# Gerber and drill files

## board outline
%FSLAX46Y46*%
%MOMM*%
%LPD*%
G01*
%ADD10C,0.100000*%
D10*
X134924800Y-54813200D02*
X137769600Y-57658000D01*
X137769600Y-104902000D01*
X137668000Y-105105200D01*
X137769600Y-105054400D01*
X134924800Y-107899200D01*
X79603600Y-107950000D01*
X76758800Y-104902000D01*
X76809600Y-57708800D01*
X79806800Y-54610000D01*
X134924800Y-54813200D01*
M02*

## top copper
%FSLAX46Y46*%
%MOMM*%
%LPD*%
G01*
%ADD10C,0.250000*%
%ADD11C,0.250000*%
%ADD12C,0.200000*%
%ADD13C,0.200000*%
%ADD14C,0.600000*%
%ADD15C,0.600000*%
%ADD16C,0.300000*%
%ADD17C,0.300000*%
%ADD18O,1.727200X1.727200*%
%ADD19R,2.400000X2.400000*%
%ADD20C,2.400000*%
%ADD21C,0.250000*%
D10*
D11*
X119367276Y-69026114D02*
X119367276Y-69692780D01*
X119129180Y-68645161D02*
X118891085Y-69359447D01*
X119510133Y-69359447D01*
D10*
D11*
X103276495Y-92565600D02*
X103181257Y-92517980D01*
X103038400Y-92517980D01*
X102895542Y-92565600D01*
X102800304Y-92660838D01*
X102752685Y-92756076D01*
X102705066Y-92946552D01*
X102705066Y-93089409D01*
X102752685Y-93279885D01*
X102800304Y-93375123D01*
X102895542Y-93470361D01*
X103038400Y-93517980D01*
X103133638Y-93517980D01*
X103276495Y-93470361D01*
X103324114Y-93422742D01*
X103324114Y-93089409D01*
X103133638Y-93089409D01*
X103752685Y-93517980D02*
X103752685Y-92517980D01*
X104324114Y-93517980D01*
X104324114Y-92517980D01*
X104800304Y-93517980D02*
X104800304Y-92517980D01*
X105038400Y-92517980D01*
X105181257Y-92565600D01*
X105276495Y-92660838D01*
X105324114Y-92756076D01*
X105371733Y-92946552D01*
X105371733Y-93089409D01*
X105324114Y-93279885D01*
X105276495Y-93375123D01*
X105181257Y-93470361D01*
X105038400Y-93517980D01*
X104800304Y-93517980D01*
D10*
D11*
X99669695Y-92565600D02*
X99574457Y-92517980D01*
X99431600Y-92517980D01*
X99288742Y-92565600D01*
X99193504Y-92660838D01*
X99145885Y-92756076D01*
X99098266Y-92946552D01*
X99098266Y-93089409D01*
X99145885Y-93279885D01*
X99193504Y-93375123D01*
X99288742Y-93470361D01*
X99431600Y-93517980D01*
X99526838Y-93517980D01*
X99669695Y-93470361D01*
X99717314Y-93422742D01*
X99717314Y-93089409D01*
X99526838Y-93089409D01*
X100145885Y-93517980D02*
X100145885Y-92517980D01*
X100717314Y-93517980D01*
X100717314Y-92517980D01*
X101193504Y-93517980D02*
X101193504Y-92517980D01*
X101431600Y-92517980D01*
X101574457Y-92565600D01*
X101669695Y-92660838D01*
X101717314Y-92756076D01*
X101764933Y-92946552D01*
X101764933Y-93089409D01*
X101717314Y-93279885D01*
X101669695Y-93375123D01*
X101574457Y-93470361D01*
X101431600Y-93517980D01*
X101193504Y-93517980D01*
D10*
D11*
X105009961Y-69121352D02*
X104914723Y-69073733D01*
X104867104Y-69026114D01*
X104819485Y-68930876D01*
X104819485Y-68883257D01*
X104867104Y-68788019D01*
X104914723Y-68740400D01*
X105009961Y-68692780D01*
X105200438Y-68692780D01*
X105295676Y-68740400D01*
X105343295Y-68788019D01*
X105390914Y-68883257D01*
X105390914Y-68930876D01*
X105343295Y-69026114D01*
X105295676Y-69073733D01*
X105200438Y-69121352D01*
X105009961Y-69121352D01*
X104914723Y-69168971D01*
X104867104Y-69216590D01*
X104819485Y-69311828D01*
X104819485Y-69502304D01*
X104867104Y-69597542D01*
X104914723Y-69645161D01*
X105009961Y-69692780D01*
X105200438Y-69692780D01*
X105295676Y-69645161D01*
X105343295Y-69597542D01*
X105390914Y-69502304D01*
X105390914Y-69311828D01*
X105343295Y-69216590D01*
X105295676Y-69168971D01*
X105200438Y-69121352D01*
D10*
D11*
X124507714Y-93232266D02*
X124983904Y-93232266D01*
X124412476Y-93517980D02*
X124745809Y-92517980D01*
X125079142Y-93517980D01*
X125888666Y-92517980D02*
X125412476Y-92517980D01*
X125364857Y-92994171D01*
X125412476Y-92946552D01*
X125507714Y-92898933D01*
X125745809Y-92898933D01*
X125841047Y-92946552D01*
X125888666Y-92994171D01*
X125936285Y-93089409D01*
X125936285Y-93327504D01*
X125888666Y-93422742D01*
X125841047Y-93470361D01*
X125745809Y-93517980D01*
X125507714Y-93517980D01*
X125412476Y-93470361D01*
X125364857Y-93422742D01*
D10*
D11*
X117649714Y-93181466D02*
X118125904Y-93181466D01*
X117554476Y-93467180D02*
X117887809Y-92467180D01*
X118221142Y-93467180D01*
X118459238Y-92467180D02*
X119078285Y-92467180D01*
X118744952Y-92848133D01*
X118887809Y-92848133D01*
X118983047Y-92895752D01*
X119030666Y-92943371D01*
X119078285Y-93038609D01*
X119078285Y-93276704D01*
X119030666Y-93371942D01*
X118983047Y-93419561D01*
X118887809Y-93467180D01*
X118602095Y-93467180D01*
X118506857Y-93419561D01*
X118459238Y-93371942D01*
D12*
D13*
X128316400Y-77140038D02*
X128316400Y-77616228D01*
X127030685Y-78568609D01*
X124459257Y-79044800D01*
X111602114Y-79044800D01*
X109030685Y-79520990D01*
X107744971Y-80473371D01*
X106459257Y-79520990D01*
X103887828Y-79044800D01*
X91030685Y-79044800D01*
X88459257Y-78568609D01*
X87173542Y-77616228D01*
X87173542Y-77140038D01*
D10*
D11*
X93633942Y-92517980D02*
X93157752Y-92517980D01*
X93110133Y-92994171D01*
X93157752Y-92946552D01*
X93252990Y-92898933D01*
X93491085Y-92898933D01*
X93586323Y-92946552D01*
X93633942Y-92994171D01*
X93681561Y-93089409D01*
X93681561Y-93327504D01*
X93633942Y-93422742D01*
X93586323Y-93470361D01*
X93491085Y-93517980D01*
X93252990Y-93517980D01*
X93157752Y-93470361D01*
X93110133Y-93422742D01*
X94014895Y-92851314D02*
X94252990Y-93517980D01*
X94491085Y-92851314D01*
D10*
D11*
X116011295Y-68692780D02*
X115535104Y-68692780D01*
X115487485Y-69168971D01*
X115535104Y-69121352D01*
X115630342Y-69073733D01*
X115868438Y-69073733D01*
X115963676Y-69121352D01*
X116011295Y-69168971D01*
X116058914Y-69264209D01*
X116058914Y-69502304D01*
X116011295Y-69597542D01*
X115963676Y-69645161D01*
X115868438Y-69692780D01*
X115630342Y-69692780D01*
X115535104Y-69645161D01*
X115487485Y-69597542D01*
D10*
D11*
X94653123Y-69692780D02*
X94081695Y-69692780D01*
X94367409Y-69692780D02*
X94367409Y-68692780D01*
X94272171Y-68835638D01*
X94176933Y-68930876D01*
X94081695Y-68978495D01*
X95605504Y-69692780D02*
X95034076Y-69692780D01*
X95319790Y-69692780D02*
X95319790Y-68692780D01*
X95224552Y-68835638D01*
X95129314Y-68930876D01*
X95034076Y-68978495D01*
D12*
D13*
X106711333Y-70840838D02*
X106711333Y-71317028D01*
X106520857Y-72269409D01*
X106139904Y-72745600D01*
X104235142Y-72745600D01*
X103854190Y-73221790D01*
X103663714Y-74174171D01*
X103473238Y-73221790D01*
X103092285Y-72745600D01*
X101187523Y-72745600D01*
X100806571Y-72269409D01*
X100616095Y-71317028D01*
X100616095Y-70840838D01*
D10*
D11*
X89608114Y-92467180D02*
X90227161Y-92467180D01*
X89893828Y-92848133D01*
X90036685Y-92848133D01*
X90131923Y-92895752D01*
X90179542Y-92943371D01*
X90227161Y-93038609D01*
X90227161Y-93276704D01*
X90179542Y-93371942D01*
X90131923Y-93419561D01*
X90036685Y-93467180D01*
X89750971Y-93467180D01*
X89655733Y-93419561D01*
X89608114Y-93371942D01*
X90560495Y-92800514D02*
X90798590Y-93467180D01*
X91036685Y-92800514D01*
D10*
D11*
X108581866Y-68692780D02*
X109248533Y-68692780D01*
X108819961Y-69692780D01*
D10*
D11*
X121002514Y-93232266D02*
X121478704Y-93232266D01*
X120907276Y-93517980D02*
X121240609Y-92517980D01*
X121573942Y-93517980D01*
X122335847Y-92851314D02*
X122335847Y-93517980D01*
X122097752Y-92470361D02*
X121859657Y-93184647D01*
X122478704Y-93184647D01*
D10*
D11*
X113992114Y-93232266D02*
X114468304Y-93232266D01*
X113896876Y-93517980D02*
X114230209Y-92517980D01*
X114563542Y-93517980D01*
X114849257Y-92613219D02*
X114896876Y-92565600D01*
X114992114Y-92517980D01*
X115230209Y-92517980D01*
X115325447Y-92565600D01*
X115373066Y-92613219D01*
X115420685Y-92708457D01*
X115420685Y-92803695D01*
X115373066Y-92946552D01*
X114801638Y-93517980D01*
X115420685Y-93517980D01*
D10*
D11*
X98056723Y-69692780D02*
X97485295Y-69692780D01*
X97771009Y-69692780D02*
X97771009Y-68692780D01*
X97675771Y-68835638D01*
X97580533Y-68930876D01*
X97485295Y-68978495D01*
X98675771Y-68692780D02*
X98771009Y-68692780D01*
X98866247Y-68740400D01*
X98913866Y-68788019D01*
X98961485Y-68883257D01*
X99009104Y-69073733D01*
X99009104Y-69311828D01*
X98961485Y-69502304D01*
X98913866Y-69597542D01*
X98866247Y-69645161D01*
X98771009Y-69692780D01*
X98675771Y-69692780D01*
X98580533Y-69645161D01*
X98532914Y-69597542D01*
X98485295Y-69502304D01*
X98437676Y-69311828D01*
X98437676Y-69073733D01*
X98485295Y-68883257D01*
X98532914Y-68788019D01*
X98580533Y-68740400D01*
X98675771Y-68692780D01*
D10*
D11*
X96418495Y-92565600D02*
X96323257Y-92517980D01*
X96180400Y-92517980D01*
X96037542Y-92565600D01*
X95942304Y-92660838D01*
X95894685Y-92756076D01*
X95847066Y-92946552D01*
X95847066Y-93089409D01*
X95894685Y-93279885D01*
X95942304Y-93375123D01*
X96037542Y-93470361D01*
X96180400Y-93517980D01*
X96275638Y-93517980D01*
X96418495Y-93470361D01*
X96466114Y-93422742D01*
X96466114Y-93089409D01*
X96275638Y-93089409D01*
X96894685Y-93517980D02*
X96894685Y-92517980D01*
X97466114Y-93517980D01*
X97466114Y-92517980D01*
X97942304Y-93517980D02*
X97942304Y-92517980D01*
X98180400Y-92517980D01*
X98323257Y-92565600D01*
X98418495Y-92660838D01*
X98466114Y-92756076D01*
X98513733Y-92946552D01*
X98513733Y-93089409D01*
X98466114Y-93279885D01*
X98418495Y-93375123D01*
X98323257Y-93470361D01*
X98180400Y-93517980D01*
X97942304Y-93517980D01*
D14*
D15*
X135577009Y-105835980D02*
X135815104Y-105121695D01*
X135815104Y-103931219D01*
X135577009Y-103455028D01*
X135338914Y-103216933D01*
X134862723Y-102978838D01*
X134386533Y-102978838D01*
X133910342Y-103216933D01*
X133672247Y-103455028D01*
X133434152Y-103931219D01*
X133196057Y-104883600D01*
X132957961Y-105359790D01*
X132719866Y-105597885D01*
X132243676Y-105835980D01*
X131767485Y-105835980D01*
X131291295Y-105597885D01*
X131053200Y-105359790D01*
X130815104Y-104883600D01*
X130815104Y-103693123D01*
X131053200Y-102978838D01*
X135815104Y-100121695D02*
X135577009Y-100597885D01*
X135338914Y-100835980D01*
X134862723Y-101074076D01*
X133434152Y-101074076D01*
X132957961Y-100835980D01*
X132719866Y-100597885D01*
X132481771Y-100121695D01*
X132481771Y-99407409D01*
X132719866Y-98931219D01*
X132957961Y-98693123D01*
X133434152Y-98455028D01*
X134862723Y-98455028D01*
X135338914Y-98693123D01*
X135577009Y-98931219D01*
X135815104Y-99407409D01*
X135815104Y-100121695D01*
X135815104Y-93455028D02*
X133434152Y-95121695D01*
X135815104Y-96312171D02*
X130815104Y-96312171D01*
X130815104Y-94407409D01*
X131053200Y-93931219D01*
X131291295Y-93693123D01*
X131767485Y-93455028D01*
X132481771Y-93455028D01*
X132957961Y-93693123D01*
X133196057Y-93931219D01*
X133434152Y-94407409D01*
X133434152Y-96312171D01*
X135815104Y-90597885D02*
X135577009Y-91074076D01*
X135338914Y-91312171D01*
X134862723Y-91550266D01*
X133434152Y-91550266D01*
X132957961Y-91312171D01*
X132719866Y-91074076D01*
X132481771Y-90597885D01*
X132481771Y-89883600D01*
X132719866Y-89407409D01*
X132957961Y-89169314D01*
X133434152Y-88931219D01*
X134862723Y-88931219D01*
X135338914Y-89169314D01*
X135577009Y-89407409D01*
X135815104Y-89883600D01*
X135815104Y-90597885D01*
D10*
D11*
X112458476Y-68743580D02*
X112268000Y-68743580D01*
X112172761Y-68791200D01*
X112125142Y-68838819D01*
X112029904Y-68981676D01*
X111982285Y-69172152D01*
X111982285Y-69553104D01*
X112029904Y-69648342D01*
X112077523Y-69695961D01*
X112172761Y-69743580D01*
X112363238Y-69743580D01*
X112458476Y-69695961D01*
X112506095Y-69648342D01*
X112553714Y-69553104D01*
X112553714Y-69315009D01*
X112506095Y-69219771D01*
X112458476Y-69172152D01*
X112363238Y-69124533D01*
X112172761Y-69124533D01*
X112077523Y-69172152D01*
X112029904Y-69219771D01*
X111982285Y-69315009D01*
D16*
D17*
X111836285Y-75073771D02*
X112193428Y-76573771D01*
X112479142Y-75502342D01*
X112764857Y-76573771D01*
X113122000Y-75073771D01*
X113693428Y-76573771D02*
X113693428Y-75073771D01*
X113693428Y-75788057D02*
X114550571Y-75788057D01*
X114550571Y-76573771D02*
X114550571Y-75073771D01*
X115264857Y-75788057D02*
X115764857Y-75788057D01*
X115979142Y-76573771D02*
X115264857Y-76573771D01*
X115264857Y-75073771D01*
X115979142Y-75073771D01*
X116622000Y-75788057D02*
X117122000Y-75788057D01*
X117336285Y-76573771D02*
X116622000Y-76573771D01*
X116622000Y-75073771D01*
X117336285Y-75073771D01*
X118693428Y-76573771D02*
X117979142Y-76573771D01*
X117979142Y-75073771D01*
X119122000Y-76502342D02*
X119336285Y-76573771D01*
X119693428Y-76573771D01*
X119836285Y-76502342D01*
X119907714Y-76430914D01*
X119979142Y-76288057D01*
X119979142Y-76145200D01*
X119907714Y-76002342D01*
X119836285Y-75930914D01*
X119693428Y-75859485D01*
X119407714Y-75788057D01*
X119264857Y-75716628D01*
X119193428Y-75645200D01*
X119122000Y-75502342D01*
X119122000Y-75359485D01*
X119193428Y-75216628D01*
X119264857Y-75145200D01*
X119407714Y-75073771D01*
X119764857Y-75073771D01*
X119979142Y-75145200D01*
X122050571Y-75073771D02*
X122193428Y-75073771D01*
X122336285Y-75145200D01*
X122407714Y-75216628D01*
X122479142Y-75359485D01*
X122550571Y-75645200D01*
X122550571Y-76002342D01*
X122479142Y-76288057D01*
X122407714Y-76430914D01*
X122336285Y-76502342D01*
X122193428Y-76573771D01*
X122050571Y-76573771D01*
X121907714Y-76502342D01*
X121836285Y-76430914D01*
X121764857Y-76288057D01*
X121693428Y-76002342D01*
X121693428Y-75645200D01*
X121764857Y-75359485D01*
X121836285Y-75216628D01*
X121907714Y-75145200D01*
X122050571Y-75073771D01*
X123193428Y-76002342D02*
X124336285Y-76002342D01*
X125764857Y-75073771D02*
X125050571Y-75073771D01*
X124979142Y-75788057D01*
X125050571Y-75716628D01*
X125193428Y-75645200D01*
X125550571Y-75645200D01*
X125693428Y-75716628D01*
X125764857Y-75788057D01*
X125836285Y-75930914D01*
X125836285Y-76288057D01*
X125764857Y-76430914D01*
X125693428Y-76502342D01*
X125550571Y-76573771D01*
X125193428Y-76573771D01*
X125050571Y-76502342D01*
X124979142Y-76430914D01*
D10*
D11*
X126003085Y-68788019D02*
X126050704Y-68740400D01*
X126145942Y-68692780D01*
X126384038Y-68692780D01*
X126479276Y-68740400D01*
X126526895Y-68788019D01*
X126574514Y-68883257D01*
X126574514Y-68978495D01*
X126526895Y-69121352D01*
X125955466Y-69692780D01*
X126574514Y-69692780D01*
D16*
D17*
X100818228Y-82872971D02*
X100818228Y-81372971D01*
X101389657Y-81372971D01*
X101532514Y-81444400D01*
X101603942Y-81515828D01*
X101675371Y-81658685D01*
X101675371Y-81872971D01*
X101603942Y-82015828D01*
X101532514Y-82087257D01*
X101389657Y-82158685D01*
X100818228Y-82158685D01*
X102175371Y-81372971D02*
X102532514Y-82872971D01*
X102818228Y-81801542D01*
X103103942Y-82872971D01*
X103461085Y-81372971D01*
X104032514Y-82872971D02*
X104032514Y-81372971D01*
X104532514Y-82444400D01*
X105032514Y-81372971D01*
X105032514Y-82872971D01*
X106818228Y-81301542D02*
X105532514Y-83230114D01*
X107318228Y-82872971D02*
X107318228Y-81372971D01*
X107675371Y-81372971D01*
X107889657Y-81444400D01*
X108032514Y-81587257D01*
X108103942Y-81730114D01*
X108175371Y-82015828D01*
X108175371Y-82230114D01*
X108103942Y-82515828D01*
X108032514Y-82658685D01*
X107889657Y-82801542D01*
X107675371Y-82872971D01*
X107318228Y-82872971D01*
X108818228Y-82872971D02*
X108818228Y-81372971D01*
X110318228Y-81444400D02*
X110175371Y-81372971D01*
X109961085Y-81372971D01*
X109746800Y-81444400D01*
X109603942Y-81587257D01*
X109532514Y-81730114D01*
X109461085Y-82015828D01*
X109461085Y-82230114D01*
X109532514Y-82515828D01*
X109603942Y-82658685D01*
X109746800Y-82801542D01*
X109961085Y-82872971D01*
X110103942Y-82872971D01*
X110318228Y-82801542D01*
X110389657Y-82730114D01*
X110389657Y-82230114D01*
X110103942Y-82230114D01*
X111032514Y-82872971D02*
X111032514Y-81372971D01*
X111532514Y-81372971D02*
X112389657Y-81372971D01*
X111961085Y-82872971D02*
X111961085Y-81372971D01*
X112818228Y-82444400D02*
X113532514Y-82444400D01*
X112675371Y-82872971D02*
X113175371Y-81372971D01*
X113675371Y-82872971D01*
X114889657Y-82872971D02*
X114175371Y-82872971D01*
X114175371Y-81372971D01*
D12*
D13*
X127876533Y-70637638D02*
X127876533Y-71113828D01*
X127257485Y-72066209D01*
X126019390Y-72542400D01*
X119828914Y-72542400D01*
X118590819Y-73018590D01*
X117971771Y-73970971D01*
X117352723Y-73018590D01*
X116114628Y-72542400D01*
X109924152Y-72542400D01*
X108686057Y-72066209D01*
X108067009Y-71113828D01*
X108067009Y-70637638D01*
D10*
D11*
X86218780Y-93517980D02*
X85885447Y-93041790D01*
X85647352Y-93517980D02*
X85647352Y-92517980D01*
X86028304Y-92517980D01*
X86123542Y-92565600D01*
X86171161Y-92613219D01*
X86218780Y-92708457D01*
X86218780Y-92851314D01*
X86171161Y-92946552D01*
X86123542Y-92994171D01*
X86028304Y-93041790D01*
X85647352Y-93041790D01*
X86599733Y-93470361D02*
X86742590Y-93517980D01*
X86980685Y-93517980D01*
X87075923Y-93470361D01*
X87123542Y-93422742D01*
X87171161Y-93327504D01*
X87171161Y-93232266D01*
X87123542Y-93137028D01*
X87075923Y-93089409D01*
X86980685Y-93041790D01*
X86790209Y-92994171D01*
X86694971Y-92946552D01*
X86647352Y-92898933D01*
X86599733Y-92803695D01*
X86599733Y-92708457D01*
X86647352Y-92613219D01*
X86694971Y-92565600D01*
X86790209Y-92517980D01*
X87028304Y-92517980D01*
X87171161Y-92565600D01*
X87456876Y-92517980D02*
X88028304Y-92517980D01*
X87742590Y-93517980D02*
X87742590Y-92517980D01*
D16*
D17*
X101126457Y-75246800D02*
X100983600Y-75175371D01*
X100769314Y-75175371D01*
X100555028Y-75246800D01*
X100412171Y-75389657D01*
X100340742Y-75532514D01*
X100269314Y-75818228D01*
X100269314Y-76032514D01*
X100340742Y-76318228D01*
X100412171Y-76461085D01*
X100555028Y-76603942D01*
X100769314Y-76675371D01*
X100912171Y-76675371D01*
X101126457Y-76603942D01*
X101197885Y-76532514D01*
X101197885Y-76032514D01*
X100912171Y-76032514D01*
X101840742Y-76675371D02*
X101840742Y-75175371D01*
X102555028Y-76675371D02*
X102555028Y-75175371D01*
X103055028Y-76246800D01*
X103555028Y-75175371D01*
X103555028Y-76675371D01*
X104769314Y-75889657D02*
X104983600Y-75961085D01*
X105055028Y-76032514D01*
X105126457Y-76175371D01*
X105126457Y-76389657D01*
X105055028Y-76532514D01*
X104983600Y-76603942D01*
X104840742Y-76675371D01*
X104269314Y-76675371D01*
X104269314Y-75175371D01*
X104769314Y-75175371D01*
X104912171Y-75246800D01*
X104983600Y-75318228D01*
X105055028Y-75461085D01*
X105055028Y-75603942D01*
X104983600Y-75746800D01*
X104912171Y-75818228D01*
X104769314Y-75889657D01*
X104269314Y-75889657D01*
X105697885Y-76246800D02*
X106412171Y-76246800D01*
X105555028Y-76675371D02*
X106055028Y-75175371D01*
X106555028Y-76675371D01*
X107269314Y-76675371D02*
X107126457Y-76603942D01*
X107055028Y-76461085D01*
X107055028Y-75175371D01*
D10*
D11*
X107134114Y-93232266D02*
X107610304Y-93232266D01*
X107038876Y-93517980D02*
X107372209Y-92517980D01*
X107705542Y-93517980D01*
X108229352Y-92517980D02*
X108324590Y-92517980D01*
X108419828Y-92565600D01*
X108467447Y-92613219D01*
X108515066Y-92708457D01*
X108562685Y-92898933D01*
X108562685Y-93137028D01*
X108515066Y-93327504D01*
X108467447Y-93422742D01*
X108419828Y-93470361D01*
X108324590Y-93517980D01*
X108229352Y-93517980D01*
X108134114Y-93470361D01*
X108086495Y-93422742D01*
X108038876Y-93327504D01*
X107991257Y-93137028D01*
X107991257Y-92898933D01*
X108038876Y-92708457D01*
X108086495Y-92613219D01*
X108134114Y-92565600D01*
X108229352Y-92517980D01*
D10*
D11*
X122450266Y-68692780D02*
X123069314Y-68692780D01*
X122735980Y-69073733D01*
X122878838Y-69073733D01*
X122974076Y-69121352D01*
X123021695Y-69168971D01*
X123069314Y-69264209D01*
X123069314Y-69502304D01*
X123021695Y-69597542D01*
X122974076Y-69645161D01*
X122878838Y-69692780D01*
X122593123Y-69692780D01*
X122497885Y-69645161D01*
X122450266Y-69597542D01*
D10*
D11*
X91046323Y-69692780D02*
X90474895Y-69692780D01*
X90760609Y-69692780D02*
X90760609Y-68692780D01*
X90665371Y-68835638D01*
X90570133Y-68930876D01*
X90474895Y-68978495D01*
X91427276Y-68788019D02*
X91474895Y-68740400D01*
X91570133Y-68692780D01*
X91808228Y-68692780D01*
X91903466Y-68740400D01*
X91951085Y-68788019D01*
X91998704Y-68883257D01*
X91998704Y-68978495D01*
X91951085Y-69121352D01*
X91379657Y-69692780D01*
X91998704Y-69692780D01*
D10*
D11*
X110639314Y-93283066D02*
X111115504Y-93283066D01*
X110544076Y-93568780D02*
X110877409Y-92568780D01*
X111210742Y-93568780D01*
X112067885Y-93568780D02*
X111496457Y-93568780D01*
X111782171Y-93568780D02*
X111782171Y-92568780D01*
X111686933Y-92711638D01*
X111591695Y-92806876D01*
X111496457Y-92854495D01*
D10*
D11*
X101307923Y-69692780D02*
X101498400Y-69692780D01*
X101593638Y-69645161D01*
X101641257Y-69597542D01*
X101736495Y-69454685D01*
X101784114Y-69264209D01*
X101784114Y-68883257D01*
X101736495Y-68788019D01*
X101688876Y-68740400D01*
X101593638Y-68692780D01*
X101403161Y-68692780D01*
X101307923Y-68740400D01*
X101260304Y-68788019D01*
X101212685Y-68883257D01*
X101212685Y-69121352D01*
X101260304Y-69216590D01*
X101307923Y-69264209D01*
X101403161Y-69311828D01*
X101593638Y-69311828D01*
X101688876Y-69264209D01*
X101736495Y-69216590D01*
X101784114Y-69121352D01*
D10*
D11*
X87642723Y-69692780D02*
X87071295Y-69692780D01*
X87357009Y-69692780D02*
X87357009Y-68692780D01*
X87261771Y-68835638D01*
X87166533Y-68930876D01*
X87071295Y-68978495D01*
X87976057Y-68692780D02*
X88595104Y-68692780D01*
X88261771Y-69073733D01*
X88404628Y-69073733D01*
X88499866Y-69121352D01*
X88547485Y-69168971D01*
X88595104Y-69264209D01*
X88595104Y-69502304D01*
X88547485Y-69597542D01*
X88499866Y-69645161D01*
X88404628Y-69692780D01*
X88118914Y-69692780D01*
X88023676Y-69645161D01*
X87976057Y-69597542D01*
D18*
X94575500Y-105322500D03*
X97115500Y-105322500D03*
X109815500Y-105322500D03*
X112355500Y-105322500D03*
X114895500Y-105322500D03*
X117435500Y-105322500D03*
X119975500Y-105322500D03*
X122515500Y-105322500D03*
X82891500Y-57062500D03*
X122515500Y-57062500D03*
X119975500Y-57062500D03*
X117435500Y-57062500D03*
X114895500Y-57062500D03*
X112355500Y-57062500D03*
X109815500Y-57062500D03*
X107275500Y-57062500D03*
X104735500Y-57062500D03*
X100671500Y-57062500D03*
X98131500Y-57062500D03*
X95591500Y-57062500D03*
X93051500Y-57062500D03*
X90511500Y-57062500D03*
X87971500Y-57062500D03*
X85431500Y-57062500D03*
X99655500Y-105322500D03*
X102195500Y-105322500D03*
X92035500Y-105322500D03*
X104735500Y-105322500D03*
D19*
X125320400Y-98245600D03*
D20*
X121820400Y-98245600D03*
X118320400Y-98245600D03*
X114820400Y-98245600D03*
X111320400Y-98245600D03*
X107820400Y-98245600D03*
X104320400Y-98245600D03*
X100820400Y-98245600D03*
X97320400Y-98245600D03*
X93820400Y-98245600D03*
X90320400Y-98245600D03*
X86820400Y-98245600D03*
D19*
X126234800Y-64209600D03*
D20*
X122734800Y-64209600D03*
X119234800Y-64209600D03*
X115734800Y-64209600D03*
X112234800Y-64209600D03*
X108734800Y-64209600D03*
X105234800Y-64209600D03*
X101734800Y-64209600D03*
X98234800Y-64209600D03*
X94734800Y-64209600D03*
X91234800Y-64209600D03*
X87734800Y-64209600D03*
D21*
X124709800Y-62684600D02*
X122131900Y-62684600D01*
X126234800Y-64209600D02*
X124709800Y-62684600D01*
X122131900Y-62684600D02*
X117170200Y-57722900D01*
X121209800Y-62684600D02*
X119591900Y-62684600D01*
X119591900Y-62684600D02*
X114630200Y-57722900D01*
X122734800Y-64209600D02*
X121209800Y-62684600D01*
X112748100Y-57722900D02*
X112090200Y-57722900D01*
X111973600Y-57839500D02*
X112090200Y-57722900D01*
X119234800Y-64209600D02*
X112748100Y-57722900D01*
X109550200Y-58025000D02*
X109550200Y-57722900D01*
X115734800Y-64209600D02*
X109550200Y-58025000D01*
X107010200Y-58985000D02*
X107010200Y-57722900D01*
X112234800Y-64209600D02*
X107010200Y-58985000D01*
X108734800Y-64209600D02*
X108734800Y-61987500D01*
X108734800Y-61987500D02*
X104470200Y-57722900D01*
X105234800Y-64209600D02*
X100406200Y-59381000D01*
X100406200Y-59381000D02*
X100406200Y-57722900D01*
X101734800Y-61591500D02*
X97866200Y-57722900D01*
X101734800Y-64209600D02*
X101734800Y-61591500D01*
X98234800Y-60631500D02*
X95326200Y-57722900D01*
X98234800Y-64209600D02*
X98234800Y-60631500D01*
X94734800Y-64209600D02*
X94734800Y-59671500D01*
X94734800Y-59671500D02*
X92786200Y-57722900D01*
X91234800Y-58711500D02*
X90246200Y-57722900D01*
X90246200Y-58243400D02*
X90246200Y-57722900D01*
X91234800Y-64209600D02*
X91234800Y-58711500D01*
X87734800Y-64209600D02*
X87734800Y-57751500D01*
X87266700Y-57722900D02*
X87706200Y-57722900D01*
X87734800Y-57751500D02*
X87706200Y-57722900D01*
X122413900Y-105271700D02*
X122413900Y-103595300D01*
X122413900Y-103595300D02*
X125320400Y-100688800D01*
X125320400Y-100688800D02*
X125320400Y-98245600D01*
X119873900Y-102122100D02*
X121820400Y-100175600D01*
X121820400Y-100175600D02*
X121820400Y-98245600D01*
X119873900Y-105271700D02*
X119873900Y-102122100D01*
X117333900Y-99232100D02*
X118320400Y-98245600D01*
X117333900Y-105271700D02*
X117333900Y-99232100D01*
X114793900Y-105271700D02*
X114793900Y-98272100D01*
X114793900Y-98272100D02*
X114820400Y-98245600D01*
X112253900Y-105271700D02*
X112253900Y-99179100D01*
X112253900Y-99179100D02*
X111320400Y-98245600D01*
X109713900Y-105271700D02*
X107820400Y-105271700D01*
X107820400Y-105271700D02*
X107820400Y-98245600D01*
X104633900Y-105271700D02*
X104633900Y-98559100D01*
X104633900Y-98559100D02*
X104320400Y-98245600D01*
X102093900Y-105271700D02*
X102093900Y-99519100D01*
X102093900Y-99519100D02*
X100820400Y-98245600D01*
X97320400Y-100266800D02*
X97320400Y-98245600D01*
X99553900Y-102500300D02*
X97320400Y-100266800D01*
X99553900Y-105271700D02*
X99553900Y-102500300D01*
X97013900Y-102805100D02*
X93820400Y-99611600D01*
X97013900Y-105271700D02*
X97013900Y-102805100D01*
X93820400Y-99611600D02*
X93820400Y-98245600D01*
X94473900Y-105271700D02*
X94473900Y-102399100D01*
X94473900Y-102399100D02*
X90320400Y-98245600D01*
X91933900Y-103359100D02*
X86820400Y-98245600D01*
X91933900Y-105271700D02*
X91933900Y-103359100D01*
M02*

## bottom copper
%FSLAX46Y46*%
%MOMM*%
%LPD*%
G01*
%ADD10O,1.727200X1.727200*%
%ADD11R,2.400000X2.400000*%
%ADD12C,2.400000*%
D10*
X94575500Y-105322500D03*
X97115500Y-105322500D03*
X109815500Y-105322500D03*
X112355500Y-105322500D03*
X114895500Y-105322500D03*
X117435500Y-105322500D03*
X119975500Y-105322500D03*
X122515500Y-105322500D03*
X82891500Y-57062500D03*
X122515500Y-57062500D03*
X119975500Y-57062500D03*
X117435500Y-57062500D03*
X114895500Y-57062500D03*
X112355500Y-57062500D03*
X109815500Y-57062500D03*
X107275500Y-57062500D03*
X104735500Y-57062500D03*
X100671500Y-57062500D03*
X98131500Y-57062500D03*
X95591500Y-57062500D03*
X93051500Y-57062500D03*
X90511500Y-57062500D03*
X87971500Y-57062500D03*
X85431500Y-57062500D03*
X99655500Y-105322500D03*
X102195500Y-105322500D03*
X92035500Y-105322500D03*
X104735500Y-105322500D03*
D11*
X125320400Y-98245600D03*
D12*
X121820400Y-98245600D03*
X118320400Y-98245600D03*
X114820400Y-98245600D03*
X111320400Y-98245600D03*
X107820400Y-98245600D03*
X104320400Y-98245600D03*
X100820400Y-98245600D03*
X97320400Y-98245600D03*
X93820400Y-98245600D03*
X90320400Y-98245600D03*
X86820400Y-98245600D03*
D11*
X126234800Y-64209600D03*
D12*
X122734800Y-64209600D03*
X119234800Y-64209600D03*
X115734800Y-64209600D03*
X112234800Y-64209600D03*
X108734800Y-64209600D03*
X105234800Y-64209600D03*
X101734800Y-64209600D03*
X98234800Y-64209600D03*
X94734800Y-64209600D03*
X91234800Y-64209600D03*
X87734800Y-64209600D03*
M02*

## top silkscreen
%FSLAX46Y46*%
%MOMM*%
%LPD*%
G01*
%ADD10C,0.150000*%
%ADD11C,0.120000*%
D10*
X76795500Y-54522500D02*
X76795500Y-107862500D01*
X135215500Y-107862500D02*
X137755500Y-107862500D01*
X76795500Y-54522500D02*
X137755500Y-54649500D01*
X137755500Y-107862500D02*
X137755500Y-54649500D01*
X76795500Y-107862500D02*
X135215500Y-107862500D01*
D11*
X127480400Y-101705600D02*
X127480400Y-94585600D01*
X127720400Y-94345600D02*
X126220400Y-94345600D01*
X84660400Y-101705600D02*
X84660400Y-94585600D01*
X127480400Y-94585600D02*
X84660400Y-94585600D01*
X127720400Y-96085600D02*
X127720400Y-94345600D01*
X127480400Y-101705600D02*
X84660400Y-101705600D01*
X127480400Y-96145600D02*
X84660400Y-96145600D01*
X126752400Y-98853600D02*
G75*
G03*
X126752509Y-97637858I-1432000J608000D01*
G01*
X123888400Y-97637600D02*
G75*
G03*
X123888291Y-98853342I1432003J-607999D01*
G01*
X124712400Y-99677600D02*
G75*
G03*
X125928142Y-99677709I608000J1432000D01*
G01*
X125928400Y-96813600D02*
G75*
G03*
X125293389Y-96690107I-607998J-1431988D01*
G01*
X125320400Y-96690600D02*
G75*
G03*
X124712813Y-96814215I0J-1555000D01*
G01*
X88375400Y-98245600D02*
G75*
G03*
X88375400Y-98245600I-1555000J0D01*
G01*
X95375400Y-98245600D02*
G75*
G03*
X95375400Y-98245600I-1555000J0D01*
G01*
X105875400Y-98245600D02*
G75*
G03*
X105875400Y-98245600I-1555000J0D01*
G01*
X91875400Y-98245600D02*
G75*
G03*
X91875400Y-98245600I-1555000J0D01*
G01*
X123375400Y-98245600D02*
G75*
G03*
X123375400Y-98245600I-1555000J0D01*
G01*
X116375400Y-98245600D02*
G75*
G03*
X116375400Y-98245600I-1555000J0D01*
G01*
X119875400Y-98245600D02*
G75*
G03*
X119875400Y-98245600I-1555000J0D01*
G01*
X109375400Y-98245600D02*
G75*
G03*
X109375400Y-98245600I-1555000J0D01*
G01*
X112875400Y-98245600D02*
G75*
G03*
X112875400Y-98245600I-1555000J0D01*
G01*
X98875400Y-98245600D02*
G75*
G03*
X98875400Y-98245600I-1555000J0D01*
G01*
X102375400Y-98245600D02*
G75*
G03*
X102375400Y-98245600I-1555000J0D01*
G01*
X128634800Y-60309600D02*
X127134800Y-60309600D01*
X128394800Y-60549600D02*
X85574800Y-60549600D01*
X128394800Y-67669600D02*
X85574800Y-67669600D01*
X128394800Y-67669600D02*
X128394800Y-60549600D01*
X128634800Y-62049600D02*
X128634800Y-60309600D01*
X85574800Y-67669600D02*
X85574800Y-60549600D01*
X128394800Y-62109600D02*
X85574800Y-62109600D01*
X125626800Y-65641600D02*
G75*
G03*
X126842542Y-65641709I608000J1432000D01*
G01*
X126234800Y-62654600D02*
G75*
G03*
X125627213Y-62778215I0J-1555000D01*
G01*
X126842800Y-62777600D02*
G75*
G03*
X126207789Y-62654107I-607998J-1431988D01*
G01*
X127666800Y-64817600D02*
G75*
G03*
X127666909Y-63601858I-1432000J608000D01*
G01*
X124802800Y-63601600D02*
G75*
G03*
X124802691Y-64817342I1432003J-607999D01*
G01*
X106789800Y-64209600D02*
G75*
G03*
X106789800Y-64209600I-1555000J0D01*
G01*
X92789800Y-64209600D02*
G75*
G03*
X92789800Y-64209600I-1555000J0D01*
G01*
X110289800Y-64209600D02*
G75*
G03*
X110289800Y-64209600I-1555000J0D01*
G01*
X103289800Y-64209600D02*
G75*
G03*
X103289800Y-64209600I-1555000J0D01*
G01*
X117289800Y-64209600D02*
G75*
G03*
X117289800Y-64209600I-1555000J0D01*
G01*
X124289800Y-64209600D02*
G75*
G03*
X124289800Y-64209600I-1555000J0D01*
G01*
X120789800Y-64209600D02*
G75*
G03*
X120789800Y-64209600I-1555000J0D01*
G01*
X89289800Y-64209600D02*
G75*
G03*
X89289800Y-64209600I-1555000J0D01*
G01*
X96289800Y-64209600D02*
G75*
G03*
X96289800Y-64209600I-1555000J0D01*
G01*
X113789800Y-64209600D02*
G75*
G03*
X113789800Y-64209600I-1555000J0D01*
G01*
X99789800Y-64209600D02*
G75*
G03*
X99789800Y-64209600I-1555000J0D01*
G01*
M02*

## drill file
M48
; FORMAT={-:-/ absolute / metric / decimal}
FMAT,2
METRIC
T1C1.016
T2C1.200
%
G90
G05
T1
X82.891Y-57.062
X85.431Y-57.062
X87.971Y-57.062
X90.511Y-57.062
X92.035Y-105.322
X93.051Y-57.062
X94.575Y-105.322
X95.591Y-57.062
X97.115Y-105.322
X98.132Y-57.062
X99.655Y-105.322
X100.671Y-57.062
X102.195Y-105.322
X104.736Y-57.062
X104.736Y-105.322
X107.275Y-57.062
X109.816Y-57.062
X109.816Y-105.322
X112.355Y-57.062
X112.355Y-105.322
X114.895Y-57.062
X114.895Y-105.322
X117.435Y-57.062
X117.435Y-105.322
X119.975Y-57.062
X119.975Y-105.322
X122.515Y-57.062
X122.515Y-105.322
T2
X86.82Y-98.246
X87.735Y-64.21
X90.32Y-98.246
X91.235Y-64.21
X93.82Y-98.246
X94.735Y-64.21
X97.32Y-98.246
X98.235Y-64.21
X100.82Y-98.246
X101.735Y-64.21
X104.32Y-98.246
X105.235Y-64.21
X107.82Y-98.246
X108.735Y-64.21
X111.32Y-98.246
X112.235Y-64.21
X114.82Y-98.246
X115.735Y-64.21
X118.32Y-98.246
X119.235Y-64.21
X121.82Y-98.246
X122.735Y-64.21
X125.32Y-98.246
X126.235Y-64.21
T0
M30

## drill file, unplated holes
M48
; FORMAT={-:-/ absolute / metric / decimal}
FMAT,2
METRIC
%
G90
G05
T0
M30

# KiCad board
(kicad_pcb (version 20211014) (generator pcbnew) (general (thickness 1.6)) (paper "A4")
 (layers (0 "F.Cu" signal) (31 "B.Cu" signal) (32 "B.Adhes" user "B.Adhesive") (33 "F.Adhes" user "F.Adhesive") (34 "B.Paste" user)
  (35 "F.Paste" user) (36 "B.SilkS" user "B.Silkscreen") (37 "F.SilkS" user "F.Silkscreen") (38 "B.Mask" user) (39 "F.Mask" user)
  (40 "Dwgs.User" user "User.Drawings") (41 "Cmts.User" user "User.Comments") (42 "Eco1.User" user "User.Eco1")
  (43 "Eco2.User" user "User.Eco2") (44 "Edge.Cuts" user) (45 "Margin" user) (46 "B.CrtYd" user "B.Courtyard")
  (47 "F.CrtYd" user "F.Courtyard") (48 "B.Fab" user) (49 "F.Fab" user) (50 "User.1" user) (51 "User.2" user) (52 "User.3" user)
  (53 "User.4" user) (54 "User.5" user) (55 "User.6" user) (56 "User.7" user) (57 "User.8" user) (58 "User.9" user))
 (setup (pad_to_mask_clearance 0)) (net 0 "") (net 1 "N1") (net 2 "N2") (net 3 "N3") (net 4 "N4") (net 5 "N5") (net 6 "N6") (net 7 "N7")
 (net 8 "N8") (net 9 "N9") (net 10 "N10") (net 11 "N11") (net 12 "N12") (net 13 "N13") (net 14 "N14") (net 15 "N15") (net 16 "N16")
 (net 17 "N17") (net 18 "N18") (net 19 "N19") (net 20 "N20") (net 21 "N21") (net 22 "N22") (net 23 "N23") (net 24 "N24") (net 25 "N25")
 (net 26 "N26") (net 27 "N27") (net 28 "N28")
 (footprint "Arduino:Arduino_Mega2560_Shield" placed (layer "F.Cu") (at 59.0155 107.8625)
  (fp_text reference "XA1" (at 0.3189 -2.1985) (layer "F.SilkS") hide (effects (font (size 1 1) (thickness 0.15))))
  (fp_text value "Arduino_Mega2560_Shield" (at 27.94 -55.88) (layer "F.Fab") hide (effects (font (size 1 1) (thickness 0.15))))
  (fp_line (start 17.78 -53.34) (end 17.78 0) (layer "F.SilkS") (width 0.15))
  (fp_line (start 76.2 0) (end 78.74 0) (layer "F.SilkS") (width 0.15))
  (fp_line (start 17.78 -53.34) (end 78.74 -53.213) (layer "F.SilkS") (width 0.15))
  (fp_line (start 78.74 0) (end 78.74 -53.213) (layer "F.SilkS") (width 0.15))
  (fp_line (start 17.78 0) (end 76.2 0) (layer "F.SilkS") (width 0.15))
  (pad "3V3" thru_hole oval (at 35.56 -2.54) (size 1.7272 1.7272) (drill 1.016) (layers *.Cu *.Mask) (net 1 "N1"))
  (pad "5V1" thru_hole oval (at 38.1 -2.54) (size 1.7272 1.7272) (drill 1.016) (layers *.Cu *.Mask) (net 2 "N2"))
  (pad "A0" thru_hole oval (at 50.8 -2.54) (size 1.7272 1.7272) (drill 1.016) (layers *.Cu *.Mask) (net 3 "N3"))
  (pad "A1" thru_hole oval (at 53.34 -2.54) (size 1.7272 1.7272) (drill 1.016) (layers *.Cu *.Mask) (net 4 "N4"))
  (pad "A2" thru_hole oval (at 55.88 -2.54) (size 1.7272 1.7272) (drill 1.016) (layers *.Cu *.Mask) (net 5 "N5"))
  (pad "A3" thru_hole oval (at 58.42 -2.54) (size 1.7272 1.7272) (drill 1.016) (layers *.Cu *.Mask) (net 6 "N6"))
  (pad "A4" thru_hole oval (at 60.96 -2.54) (size 1.7272 1.7272) (drill 1.016) (layers *.Cu *.Mask) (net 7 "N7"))
  (pad "A5" thru_hole oval (at 63.5 -2.54) (size 1.7272 1.7272) (drill 1.016) (layers *.Cu *.Mask) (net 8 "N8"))
  (pad "AREF" thru_hole oval (at 23.876 -50.8) (size 1.7272 1.7272) (drill 1.016) (layers *.Cu *.Mask) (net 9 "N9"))
  (pad "D0" thru_hole oval (at 63.5 -50.8) (size 1.7272 1.7272) (drill 1.016) (layers *.Cu *.Mask) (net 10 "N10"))
  (pad "D1" thru_hole oval (at 60.96 -50.8) (size 1.7272 1.7272) (drill 1.016) (layers *.Cu *.Mask) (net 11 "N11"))
  (pad "D2" thru_hole oval (at 58.42 -50.8) (size 1.7272 1.7272) (drill 1.016) (layers *.Cu *.Mask) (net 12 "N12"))
  (pad "D3" thru_hole oval (at 55.88 -50.8) (size 1.7272 1.7272) (drill 1.016) (layers *.Cu *.Mask) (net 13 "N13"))
  (pad "D4" thru_hole oval (at 53.34 -50.8) (size 1.7272 1.7272) (drill 1.016) (layers *.Cu *.Mask) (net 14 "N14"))
  (pad "D5" thru_hole oval (at 50.8 -50.8) (size 1.7272 1.7272) (drill 1.016) (layers *.Cu *.Mask) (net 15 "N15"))
  (pad "D6" thru_hole oval (at 48.26 -50.8) (size 1.7272 1.7272) (drill 1.016) (layers *.Cu *.Mask) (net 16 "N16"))
  (pad "D7" thru_hole oval (at 45.72 -50.8) (size 1.7272 1.7272) (drill 1.016) (layers *.Cu *.Mask) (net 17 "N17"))
  (pad "D8" thru_hole oval (at 41.656 -50.8) (size 1.7272 1.7272) (drill 1.016) (layers *.Cu *.Mask) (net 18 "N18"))
  (pad "D9" thru_hole oval (at 39.116 -50.8) (size 1.7272 1.7272) (drill 1.016) (layers *.Cu *.Mask) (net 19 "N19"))
  (pad "D10" thru_hole oval (at 36.576 -50.8) (size 1.7272 1.7272) (drill 1.016) (layers *.Cu *.Mask) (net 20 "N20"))
  (pad "D11" thru_hole oval (at 34.036 -50.8) (size 1.7272 1.7272) (drill 1.016) (layers *.Cu *.Mask) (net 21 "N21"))
  (pad "D12" thru_hole oval (at 31.496 -50.8) (size 1.7272 1.7272) (drill 1.016) (layers *.Cu *.Mask) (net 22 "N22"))
  (pad "D13" thru_hole oval (at 28.956 -50.8) (size 1.7272 1.7272) (drill 1.016) (layers *.Cu *.Mask) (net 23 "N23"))
  (pad "GND1" thru_hole oval (at 26.416 -50.8) (size 1.7272 1.7272) (drill 1.016) (layers *.Cu *.Mask) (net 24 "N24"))
  (pad "GND2" thru_hole oval (at 40.64 -2.54) (size 1.7272 1.7272) (drill 1.016) (layers *.Cu *.Mask) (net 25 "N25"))
  (pad "GND3" thru_hole oval (at 43.18 -2.54) (size 1.7272 1.7272) (drill 1.016) (layers *.Cu *.Mask) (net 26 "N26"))
  (pad "RST1" thru_hole oval (at 33.02 -2.54) (size 1.7272 1.7272) (drill 1.016) (layers *.Cu *.Mask) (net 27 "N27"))
  (pad "VIN" thru_hole oval (at 45.72 -2.54) (size 1.7272 1.7272) (drill 1.016) (layers *.Cu *.Mask) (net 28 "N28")))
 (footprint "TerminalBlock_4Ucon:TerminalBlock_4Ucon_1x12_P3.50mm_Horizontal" (layer "F.Cu") (at 125.3204 98.2456 180)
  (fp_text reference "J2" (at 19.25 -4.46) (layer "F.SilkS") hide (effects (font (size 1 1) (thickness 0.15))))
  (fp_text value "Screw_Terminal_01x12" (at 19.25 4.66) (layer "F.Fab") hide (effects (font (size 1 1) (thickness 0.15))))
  (fp_line (start -2.16 -3.46) (end -2.16 3.66) (layer "F.SilkS") (width 0.12))
  (fp_line (start -2.4 3.9) (end -0.9 3.9) (layer "F.SilkS") (width 0.12))
  (fp_line (start 40.66 -3.46) (end 40.66 3.66) (layer "F.SilkS") (width 0.12))
  (fp_line (start -2.16 3.66) (end 40.66 3.66) (layer "F.SilkS") (width 0.12))
  (fp_line (start -2.4 2.16) (end -2.4 3.9) (layer "F.SilkS") (width 0.12))
  (fp_line (start -2.16 -3.46) (end 40.66 -3.46) (layer "F.SilkS") (width 0.12))
  (fp_line (start -2.16 2.1) (end 40.66 2.1) (layer "F.SilkS") (width 0.12))
  (fp_arc (start -1.432109 0.607742) (mid -1.555727 -0.00014) (end -1.432 -0.608) (layer "F.SilkS") (width 0.12))
  (fp_arc (start 1.432109 -0.607742) (mid 1.555727 0.00014) (end 1.432 0.608) (layer "F.SilkS") (width 0.12))
  (fp_arc (start -0.607742 -1.432109) (mid 0.00014 -1.555727) (end 0.608 -1.432) (layer "F.SilkS") (width 0.12))
  (fp_arc (start 0.027011 1.555493) (mid -0.296984 1.527118) (end -0.608 1.432) (layer "F.SilkS") (width 0.12))
  (fp_arc (start 0.607587 1.431385) (mid 0.310017 1.523783) (end 0 1.555) (layer "F.SilkS") (width 0.12))
  (fp_circle (center 38.5 0) (end 40.055 0) (layer "F.SilkS") (width 0.12) (fill none))
  (fp_circle (center 31.5 0) (end 33.055 0) (layer "F.SilkS") (width 0.12) (fill none))
  (fp_circle (center 21 0) (end 22.555 0) (layer "F.SilkS") (width 0.12) (fill none))
  (fp_circle (center 35 0) (end 36.555 0) (layer "F.SilkS") (width 0.12) (fill none))
  (fp_circle (center 3.5 0) (end 5.055 0) (layer "F.SilkS") (width 0.12) (fill none))
  (fp_circle (center 10.5 0) (end 12.055 0) (layer "F.SilkS") (width 0.12) (fill none))
  (fp_circle (center 7 0) (end 8.555 0) (layer "F.SilkS") (width 0.12) (fill none))
  (fp_circle (center 17.5 0) (end 19.055 0) (layer "F.SilkS") (width 0.12) (fill none))
  (fp_circle (center 14 0) (end 15.555 0) (layer "F.SilkS") (width 0.12) (fill none))
  (fp_circle (center 28 0) (end 29.555 0) (layer "F.SilkS") (width 0.12) (fill none))
  (fp_circle (center 24.5 0) (end 26.055 0) (layer "F.SilkS") (width 0.12) (fill none))
  (pad "1" thru_hole rect (at 0 0 180) (size 2.4 2.4) (drill 1.2) (layers *.Cu *.Mask) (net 8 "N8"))
  (pad "2" thru_hole circle (at 3.5 0 180) (size 2.4 2.4) (drill 1.2) (layers *.Cu *.Mask) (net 7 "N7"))
  (pad "3" thru_hole circle (at 7 0 180) (size 2.4 2.4) (drill 1.2) (layers *.Cu *.Mask) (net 6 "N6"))
  (pad "4" thru_hole circle (at 10.5 0 180) (size 2.4 2.4) (drill 1.2) (layers *.Cu *.Mask) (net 5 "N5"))
  (pad "5" thru_hole circle (at 14 0 180) (size 2.4 2.4) (drill 1.2) (layers *.Cu *.Mask) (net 4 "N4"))
  (pad "6" thru_hole circle (at 17.5 0 180) (size 2.4 2.4) (drill 1.2) (layers *.Cu *.Mask) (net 3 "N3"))
  (pad "7" thru_hole circle (at 21 0 180) (size 2.4 2.4) (drill 1.2) (layers *.Cu *.Mask) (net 28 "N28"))
  (pad "8" thru_hole circle (at 24.5 0 180) (size 2.4 2.4) (drill 1.2) (layers *.Cu *.Mask) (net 26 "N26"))
  (pad "9" thru_hole circle (at 28 0 180) (size 2.4 2.4) (drill 1.2) (layers *.Cu *.Mask) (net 25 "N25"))
  (pad "10" thru_hole circle (at 31.5 0 180) (size 2.4 2.4) (drill 1.2) (layers *.Cu *.Mask) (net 2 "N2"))
  (pad "11" thru_hole circle (at 35 0 180) (size 2.4 2.4) (drill 1.2) (layers *.Cu *.Mask) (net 1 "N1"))
  (pad "12" thru_hole circle (at 38.5 0 180) (size 2.4 2.4) (drill 1.2) (layers *.Cu *.Mask) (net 27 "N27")))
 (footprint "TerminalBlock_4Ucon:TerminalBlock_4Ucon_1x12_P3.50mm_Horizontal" (layer "F.Cu") (at 126.2348 64.2096 180)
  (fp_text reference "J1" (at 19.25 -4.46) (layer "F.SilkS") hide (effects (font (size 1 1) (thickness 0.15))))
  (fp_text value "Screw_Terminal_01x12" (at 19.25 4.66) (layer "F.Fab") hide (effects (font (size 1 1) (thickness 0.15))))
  (fp_line (start -2.4 3.9) (end -0.9 3.9) (layer "F.SilkS") (width 0.12))
  (fp_line (start -2.16 3.66) (end 40.66 3.66) (layer "F.SilkS") (width 0.12))
  (fp_line (start -2.16 -3.46) (end 40.66 -3.46) (layer "F.SilkS") (width 0.12))
  (fp_line (start -2.16 -3.46) (end -2.16 3.66) (layer "F.SilkS") (width 0.12))
  (fp_line (start -2.4 2.16) (end -2.4 3.9) (layer "F.SilkS") (width 0.12))
  (fp_line (start 40.66 -3.46) (end 40.66 3.66) (layer "F.SilkS") (width 0.12))
  (fp_line (start -2.16 2.1) (end 40.66 2.1) (layer "F.SilkS") (width 0.12))
  (fp_arc (start -0.607742 -1.432109) (mid 0.00014 -1.555727) (end 0.608 -1.432) (layer "F.SilkS") (width 0.12))
  (fp_arc (start 0.607587 1.431385) (mid 0.310017 1.523783) (end 0 1.555) (layer "F.SilkS") (width 0.12))
  (fp_arc (start 0.027011 1.555493) (mid -0.296984 1.527118) (end -0.608 1.432) (layer "F.SilkS") (width 0.12))
  (fp_arc (start -1.432109 0.607742) (mid -1.555727 -0.00014) (end -1.432 -0.608) (layer "F.SilkS") (width 0.12))
  (fp_arc (start 1.432109 -0.607742) (mid 1.555727 0.00014) (end 1.432 0.608) (layer "F.SilkS") (width 0.12))
  (fp_circle (center 21 0) (end 22.555 0) (layer "F.SilkS") (width 0.12) (fill none))
  (fp_circle (center 35 0) (end 36.555 0) (layer "F.SilkS") (width 0.12) (fill none))
  (fp_circle (center 17.5 0) (end 19.055 0) (layer "F.SilkS") (width 0.12) (fill none))
  (fp_circle (center 24.5 0) (end 26.055 0) (layer "F.SilkS") (width 0.12) (fill none))
  (fp_circle (center 10.5 0) (end 12.055 0) (layer "F.SilkS") (width 0.12) (fill none))
  (fp_circle (center 3.5 0) (end 5.055 0) (layer "F.SilkS") (width 0.12) (fill none))
  (fp_circle (center 7 0) (end 8.555 0) (layer "F.SilkS") (width 0.12) (fill none))
  (fp_circle (center 38.5 0) (end 40.055 0) (layer "F.SilkS") (width 0.12) (fill none))
  (fp_circle (center 31.5 0) (end 33.055 0) (layer "F.SilkS") (width 0.12) (fill none))
  (fp_circle (center 14 0) (end 15.555 0) (layer "F.SilkS") (width 0.12) (fill none))
  (fp_circle (center 28 0) (end 29.555 0) (layer "F.SilkS") (width 0.12) (fill none))
  (pad "1" thru_hole rect (at 0 0 180) (size 2.4 2.4) (drill 1.2) (layers *.Cu *.Mask) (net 12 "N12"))
  (pad "2" thru_hole circle (at 3.5 0 180) (size 2.4 2.4) (drill 1.2) (layers *.Cu *.Mask) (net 13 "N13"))
  (pad "3" thru_hole circle (at 7 0 180) (size 2.4 2.4) (drill 1.2) (layers *.Cu *.Mask) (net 14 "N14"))
  (pad "4" thru_hole circle (at 10.5 0 180) (size 2.4 2.4) (drill 1.2) (layers *.Cu *.Mask) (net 15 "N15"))
  (pad "5" thru_hole circle (at 14 0 180) (size 2.4 2.4) (drill 1.2) (layers *.Cu *.Mask) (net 16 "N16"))
  (pad "6" thru_hole circle (at 17.5 0 180) (size 2.4 2.4) (drill 1.2) (layers *.Cu *.Mask) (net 17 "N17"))
  (pad "7" thru_hole circle (at 21 0 180) (size 2.4 2.4) (drill 1.2) (layers *.Cu *.Mask) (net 18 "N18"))
  (pad "8" thru_hole circle (at 24.5 0 180) (size 2.4 2.4) (drill 1.2) (layers *.Cu *.Mask) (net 19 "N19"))
  (pad "9" thru_hole circle (at 28 0 180) (size 2.4 2.4) (drill 1.2) (layers *.Cu *.Mask) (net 20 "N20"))
  (pad "10" thru_hole circle (at 31.5 0 180) (size 2.4 2.4) (drill 1.2) (layers *.Cu *.Mask) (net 21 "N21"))
  (pad "11" thru_hole circle (at 35 0 180) (size 2.4 2.4) (drill 1.2) (layers *.Cu *.Mask) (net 22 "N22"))
  (pad "12" thru_hole circle (at 38.5 0 180) (size 2.4 2.4) (drill 1.2) (layers *.Cu *.Mask) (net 23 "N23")))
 (gr_poly
  (pts (xy 134.9248 54.8132) (xy 137.7696 57.658) (xy 137.7696 104.902) (xy 137.668 105.1052) (xy 137.7696 105.0544) (xy 134.9248 107.8992)
   (xy 79.6036 107.95) (xy 76.7588 104.902) (xy 76.8096 57.7088) (xy 79.8068 54.61))
  (layer "Edge.Cuts") (width 0.1) (fill none))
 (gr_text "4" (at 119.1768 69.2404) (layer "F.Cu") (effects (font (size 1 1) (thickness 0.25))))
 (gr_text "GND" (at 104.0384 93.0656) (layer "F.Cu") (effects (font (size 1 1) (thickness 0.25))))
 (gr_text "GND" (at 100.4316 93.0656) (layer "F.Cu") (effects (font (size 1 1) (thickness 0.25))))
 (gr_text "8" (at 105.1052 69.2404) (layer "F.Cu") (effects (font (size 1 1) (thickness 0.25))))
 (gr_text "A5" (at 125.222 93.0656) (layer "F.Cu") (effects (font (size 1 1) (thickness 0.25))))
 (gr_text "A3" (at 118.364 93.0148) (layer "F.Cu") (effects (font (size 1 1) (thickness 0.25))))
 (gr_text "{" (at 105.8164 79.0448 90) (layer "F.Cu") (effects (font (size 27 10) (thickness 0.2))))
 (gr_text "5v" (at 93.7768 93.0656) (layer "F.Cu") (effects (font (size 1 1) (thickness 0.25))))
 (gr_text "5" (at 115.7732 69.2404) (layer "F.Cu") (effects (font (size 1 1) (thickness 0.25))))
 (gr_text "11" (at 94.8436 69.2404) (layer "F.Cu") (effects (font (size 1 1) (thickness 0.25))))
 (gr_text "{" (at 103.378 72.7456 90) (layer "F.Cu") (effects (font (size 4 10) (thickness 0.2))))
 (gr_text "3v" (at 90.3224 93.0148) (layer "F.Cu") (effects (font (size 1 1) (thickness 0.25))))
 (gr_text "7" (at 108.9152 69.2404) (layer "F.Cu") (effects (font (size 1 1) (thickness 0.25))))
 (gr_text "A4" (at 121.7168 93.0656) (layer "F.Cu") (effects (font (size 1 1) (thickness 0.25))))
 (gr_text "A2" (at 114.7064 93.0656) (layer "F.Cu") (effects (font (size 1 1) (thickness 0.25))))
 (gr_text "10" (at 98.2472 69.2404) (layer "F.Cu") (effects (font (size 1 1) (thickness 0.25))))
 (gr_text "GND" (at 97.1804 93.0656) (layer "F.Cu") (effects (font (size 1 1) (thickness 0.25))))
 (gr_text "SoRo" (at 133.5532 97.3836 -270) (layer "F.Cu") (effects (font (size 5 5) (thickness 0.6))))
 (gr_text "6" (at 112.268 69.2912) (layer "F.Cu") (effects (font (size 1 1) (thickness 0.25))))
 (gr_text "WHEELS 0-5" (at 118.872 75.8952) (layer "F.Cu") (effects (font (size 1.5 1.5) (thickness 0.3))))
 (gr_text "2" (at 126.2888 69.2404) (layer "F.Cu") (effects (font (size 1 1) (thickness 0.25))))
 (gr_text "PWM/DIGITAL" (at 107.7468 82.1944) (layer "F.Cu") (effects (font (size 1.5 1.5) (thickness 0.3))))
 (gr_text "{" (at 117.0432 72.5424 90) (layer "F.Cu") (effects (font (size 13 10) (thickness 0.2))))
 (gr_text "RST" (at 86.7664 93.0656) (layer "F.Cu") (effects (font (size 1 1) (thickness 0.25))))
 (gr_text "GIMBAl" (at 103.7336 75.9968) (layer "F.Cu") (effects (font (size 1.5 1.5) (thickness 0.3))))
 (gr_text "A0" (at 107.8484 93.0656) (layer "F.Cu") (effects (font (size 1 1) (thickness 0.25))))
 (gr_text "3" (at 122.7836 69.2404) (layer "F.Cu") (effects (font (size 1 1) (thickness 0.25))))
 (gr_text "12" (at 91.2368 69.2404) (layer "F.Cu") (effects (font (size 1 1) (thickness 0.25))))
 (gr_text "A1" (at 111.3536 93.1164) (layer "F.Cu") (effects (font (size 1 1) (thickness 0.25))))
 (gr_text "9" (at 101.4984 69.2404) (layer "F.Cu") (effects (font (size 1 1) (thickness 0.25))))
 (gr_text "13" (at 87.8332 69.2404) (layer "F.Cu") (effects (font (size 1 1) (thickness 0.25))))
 (segment (start 124.7098 62.6846) (end 122.1319 62.6846) (width 0.25) (layer "F.Cu") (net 12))
 (segment (start 126.2348 64.2096) (end 124.7098 62.6846) (width 0.25) (layer "F.Cu") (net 12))
 (segment (start 122.1319 62.6846) (end 117.1702 57.7229) (width 0.25) (layer "F.Cu") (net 12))
 (segment (start 121.2098 62.6846) (end 119.5919 62.6846) (width 0.25) (layer "F.Cu") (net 13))
 (segment (start 119.5919 62.6846) (end 114.6302 57.7229) (width 0.25) (layer "F.Cu") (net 13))
 (segment (start 122.7348 64.2096) (end 121.2098 62.6846) (width 0.25) (layer "F.Cu") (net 13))
 (segment (start 112.7481 57.7229) (end 112.0902 57.7229) (width 0.25) (layer "F.Cu") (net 14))
 (segment (start 111.9736 57.8395) (end 112.0902 57.7229) (width 0.25) (layer "F.Cu") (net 14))
 (segment (start 119.2348 64.2096) (end 112.7481 57.7229) (width 0.25) (layer "F.Cu") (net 14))
 (segment (start 109.5502 58.025) (end 109.5502 57.7229) (width 0.25) (layer "F.Cu") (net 15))
 (segment (start 115.7348 64.2096) (end 109.5502 58.025) (width 0.25) (layer "F.Cu") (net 15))
 (segment (start 107.0102 58.985) (end 107.0102 57.7229) (width 0.25) (layer "F.Cu") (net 16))
 (segment (start 112.2348 64.2096) (end 107.0102 58.985) (width 0.25) (layer "F.Cu") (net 16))
 (segment (start 108.7348 64.2096) (end 108.7348 61.9875) (width 0.25) (layer "F.Cu") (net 17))
 (segment (start 108.7348 61.9875) (end 104.4702 57.7229) (width 0.25) (layer "F.Cu") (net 17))
 (segment (start 105.2348 64.2096) (end 100.4062 59.381) (width 0.25) (layer "F.Cu") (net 18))
 (segment (start 100.4062 59.381) (end 100.4062 57.7229) (width 0.25) (layer "F.Cu") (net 18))
 (segment (start 101.7348 61.5915) (end 97.8662 57.7229) (width 0.25) (layer "F.Cu") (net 19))
 (segment (start 101.7348 64.2096) (end 101.7348 61.5915) (width 0.25) (layer "F.Cu") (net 19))
 (segment (start 98.2348 60.6315) (end 95.3262 57.7229) (width 0.25) (layer "F.Cu") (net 20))
 (segment (start 98.2348 64.2096) (end 98.2348 60.6315) (width 0.25) (layer "F.Cu") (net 20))
 (segment (start 94.7348 64.2096) (end 94.7348 59.6715) (width 0.25) (layer "F.Cu") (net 21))
 (segment (start 94.7348 59.6715) (end 92.7862 57.7229) (width 0.25) (layer "F.Cu") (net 21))
 (segment (start 91.2348 58.7115) (end 90.2462 57.7229) (width 0.25) (layer "F.Cu") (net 22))
 (segment (start 90.2462 58.2434) (end 90.2462 57.7229) (width 0.25) (layer "F.Cu") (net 22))
 (segment (start 91.2348 64.2096) (end 91.2348 58.7115) (width 0.25) (layer "F.Cu") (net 22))
 (segment (start 87.7348 64.2096) (end 87.7348 57.7515) (width 0.25) (layer "F.Cu") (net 23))
 (segment (start 87.2667 57.7229) (end 87.7062 57.7229) (width 0.25) (layer "F.Cu") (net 23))
 (segment (start 87.7348 57.7515) (end 87.7062 57.7229) (width 0.25) (layer "F.Cu") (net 23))
 (segment (start 122.4139 105.2717) (end 122.4139 103.5953) (width 0.25) (layer "F.Cu") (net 8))
 (segment (start 122.4139 103.5953) (end 125.3204 100.6888) (width 0.25) (layer "F.Cu") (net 8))
 (segment (start 125.3204 100.6888) (end 125.3204 98.2456) (width 0.25) (layer "F.Cu") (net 8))
 (segment (start 119.8739 102.1221) (end 121.8204 100.1756) (width 0.25) (layer "F.Cu") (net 7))
 (segment (start 121.8204 100.1756) (end 121.8204 98.2456) (width 0.25) (layer "F.Cu") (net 7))
 (segment (start 119.8739 105.2717) (end 119.8739 102.1221) (width 0.25) (layer "F.Cu") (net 7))
 (segment (start 117.3339 99.2321) (end 118.3204 98.2456) (width 0.25) (layer "F.Cu") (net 6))
 (segment (start 117.3339 105.2717) (end 117.3339 99.2321) (width 0.25) (layer "F.Cu") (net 6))
 (segment (start 114.7939 105.2717) (end 114.7939 98.2721) (width 0.25) (layer "F.Cu") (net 5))
 (segment (start 114.7939 98.2721) (end 114.8204 98.2456) (width 0.25) (layer "F.Cu") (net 5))
 (segment (start 112.2539 105.2717) (end 112.2539 99.1791) (width 0.25) (layer "F.Cu") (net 4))
 (segment (start 112.2539 99.1791) (end 111.3204 98.2456) (width 0.25) (layer "F.Cu") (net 4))
 (segment (start 109.7139 105.2717) (end 107.8204 105.2717) (width 0.25) (layer "F.Cu") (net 3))
 (segment (start 107.8204 105.2717) (end 107.8204 98.2456) (width 0.25) (layer "F.Cu") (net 3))
 (segment (start 104.6339 105.2717) (end 104.6339 98.5591) (width 0.25) (layer "F.Cu") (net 28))
 (segment (start 104.6339 98.5591) (end 104.3204 98.2456) (width 0.25) (layer "F.Cu") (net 28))
 (segment (start 102.0939 105.2717) (end 102.0939 99.5191) (width 0.25) (layer "F.Cu") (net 26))
 (segment (start 102.0939 99.5191) (end 100.8204 98.2456) (width 0.25) (layer "F.Cu") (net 26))
 (segment (start 97.3204 100.2668) (end 97.3204 98.2456) (width 0.25) (layer "F.Cu") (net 25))
 (segment (start 99.5539 102.5003) (end 97.3204 100.2668) (width 0.25) (layer "F.Cu") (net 25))
 (segment (start 99.5539 105.2717) (end 99.5539 102.5003) (width 0.25) (layer "F.Cu") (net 25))
 (segment (start 97.0139 102.8051) (end 93.8204 99.6116) (width 0.25) (layer "F.Cu") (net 2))
 (segment (start 97.0139 105.2717) (end 97.0139 102.8051) (width 0.25) (layer "F.Cu") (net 2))
 (segment (start 93.8204 99.6116) (end 93.8204 98.2456) (width 0.25) (layer "F.Cu") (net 2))
 (segment (start 94.4739 105.2717) (end 94.4739 102.3991) (width 0.25) (layer "F.Cu") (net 1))
 (segment (start 94.4739 102.3991) (end 90.3204 98.2456) (width 0.25) (layer "F.Cu") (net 1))
 (segment (start 91.9339 103.3591) (end 86.8204 98.2456) (width 0.25) (layer "F.Cu") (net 27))
 (segment (start 91.9339 105.2717) (end 91.9339 103.3591) (width 0.25) (layer "F.Cu") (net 27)))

